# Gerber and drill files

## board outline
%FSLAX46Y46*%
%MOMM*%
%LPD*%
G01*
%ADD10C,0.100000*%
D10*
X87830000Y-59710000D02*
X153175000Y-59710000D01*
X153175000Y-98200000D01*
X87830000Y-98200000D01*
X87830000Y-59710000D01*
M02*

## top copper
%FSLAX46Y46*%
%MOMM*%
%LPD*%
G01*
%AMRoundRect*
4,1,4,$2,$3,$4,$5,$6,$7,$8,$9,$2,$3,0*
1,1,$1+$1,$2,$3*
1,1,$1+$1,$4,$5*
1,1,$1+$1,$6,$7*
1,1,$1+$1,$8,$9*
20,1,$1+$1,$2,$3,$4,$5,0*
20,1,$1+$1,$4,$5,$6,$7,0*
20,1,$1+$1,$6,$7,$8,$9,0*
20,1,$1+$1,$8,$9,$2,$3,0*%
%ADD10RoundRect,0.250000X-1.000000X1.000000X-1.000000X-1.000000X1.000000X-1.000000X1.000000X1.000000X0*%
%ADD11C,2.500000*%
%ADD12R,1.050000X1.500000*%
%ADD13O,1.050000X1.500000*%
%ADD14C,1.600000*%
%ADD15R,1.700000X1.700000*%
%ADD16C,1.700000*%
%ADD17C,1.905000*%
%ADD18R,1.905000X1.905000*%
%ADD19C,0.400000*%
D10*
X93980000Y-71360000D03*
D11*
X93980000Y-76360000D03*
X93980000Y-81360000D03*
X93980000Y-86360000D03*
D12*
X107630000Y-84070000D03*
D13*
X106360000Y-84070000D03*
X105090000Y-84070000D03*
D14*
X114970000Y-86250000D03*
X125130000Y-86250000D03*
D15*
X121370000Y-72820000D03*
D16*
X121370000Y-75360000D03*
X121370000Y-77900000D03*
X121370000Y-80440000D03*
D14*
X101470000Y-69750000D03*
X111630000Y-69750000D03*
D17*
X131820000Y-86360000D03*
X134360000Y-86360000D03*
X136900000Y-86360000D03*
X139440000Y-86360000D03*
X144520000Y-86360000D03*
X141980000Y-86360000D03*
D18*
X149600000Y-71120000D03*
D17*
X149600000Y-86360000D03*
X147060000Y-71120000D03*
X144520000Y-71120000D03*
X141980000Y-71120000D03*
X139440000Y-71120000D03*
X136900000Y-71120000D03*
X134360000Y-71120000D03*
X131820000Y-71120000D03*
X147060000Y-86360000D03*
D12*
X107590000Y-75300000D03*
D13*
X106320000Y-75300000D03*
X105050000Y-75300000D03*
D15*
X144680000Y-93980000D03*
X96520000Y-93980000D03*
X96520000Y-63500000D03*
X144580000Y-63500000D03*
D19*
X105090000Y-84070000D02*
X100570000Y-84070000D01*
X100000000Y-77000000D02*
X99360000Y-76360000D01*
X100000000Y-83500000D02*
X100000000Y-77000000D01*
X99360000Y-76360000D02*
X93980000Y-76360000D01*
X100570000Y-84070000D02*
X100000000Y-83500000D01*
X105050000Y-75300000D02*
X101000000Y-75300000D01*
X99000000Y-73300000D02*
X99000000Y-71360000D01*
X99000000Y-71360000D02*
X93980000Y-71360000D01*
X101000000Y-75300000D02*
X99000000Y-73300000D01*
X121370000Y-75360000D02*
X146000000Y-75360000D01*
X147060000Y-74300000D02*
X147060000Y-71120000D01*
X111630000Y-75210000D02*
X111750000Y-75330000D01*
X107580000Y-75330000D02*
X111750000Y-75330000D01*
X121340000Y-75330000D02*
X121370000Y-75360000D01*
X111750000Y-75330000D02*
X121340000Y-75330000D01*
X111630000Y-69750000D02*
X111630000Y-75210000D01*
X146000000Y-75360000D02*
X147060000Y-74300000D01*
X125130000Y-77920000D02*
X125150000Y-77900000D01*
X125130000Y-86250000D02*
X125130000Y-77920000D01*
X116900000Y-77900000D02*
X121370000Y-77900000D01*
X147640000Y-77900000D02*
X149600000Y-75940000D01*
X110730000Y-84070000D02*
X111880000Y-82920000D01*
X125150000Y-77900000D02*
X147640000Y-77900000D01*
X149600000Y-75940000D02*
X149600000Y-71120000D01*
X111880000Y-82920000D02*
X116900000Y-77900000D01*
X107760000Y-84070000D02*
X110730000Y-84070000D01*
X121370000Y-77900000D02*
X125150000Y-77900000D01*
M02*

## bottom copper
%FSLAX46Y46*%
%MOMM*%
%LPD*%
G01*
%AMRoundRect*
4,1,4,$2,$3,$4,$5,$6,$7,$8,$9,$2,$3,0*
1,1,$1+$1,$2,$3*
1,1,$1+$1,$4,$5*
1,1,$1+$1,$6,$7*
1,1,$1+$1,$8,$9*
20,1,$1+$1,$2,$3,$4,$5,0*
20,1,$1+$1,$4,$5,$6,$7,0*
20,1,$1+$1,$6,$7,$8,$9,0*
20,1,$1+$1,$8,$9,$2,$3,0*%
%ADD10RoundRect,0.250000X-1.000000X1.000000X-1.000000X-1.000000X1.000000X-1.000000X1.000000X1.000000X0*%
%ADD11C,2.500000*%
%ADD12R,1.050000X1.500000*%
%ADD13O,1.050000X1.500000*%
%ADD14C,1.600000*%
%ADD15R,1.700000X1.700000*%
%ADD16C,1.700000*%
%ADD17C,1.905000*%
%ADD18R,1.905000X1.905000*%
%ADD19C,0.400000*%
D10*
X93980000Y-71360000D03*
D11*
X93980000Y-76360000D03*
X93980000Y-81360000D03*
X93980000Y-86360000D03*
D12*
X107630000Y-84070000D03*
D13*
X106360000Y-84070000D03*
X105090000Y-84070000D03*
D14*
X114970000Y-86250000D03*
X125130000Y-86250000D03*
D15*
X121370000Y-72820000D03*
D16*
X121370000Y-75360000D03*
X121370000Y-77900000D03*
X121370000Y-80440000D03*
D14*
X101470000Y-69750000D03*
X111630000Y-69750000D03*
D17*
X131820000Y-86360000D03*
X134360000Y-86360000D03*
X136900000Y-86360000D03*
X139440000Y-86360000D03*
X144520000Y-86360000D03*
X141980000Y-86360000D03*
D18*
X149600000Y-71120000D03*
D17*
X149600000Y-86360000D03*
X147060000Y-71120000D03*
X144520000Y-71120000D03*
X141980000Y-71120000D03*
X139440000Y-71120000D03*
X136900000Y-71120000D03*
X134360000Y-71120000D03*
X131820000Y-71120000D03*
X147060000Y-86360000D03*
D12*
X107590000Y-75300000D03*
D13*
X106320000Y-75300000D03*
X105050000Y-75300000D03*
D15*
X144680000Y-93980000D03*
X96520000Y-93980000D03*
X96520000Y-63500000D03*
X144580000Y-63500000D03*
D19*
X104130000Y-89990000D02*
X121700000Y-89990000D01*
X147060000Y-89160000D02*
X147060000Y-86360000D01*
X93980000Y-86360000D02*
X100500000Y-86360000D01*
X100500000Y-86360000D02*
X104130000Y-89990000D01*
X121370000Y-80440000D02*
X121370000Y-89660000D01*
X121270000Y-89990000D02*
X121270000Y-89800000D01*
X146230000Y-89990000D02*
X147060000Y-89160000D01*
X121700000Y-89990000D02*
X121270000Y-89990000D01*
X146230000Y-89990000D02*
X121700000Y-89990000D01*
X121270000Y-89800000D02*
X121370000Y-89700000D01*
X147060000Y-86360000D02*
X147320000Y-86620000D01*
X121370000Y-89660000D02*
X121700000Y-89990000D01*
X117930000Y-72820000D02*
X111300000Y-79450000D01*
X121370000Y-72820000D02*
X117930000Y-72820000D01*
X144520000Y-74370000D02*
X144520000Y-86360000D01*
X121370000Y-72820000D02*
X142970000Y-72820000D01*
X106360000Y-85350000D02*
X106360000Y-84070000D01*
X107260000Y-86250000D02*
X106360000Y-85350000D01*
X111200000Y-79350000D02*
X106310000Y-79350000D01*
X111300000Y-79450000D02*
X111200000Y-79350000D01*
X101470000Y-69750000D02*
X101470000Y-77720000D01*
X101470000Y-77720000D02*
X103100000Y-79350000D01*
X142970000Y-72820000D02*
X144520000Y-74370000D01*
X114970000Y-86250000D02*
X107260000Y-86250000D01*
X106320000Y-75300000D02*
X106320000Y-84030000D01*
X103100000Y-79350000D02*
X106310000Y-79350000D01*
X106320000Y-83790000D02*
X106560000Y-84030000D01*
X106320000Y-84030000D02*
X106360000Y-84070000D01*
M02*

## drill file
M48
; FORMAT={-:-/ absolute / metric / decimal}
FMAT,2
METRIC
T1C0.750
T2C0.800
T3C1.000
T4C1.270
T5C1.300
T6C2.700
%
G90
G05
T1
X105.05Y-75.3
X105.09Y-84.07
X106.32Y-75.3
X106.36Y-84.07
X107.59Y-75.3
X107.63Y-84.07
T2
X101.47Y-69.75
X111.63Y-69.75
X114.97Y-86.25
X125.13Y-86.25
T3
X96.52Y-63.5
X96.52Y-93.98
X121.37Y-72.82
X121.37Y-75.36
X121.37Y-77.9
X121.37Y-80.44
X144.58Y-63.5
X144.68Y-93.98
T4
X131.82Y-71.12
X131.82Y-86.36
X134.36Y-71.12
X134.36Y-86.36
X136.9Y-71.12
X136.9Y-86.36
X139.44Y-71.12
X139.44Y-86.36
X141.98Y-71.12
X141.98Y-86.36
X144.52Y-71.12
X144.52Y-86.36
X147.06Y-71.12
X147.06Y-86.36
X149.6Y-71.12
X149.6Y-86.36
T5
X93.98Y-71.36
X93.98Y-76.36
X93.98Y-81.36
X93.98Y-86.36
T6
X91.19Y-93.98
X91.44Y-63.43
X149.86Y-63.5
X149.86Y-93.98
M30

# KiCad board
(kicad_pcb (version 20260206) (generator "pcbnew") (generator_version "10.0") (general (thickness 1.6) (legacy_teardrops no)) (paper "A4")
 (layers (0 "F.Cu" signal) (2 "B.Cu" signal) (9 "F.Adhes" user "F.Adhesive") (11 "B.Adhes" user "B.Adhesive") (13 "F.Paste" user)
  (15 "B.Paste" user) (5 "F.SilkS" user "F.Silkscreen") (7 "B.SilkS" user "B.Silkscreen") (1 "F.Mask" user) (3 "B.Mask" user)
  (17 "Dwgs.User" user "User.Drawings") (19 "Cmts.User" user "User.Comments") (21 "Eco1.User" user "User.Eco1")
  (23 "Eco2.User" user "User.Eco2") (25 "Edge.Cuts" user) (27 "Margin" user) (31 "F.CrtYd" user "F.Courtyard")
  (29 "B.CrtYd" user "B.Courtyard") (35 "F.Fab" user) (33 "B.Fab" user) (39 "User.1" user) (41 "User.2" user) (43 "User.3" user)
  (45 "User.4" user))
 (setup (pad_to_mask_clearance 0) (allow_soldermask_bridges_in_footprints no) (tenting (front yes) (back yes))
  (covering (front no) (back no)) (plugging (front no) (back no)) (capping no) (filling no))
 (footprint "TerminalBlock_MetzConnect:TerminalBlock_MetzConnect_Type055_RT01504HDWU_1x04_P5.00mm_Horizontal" (layer "F.Cu")
  (at 93.98 71.36 -90)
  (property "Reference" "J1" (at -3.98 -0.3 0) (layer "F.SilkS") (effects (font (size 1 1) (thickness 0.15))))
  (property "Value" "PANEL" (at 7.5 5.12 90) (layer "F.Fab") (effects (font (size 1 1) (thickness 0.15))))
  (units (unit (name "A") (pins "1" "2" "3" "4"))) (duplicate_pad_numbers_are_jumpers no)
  (pad "1" thru_hole roundrect (at 0 0 270) (size 2.5 2.5) (drill 1.3) (layers "*.Cu" "*.Mask") (remove_unused_layers no)
   (roundrect_rratio 0.1) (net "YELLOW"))
  (pad "2" thru_hole circle (at 5 0 270) (size 2.5 2.5) (drill 1.3) (layers "*.Cu" "*.Mask") (remove_unused_layers no) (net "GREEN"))
  (pad "3" thru_hole circle (at 10 0 270) (size 2.5 2.5) (drill 1.3) (layers "*.Cu" "*.Mask") (remove_unused_layers no) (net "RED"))
  (pad "4" thru_hole circle (at 15 0 270) (size 2.5 2.5) (drill 1.3) (layers "*.Cu" "*.Mask") (remove_unused_layers no) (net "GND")))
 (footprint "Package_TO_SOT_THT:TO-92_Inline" (layer "F.Cu") (at 107.63 84.07 180)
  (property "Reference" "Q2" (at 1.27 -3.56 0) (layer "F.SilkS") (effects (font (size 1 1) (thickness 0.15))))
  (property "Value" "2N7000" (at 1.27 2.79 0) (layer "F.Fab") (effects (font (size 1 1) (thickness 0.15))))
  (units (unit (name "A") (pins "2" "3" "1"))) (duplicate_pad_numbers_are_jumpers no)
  (pad "1" thru_hole rect (at 0 0 180) (size 1.05 1.5) (drill 0.75) (layers "*.Cu" "*.Mask") (remove_unused_layers no) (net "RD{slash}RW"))
  (pad "2" thru_hole oval (at 1.27 0 180) (size 1.05 1.5) (drill 0.75) (layers "*.Cu" "*.Mask") (remove_unused_layers no) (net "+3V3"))
  (pad "3" thru_hole oval (at 2.54 0 180) (size 1.05 1.5) (drill 0.75) (layers "*.Cu" "*.Mask") (remove_unused_layers no) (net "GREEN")))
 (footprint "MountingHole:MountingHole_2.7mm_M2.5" (layer "F.Cu") (at 149.86 63.5)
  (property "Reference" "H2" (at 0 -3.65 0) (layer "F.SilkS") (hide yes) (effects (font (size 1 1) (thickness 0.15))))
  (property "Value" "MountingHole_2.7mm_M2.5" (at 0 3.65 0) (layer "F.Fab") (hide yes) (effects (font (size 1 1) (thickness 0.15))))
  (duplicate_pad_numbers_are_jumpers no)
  (pad "" np_thru_hole circle (at 0 0) (size 2.7 2.7) (drill 2.7) (layers "*.Cu" "*.Mask")))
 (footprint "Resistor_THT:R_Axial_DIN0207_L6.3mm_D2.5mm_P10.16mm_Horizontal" (layer "F.Cu") (at 114.97 86.25)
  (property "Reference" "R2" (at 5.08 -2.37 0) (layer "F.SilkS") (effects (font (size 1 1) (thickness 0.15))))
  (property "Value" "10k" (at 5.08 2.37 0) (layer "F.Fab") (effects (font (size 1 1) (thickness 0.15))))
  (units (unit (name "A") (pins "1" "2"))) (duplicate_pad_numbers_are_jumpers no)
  (pad "1" thru_hole circle (at 0 0) (size 1.6 1.6) (drill 0.8) (layers "*.Cu" "*.Mask") (remove_unused_layers no) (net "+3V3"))
  (pad "2" thru_hole circle (at 10.16 0) (size 1.6 1.6) (drill 0.8) (layers "*.Cu" "*.Mask") (remove_unused_layers no) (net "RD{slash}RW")))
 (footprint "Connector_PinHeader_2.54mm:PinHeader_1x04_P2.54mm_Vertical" (layer "F.Cu") (at 121.37 72.82)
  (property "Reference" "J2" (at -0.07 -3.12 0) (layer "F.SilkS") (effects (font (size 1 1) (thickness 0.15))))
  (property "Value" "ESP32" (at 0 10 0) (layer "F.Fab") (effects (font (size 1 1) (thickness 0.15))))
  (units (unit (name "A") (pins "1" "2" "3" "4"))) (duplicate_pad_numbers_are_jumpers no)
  (pad "1" thru_hole rect (at 0 0) (size 1.7 1.7) (drill 1) (layers "*.Cu" "*.Mask") (remove_unused_layers no) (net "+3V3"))
  (pad "2" thru_hole circle (at 0 2.54) (size 1.7 1.7) (drill 1) (layers "*.Cu" "*.Mask") (remove_unused_layers no) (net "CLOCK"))
  (pad "3" thru_hole circle (at 0 5.08) (size 1.7 1.7) (drill 1) (layers "*.Cu" "*.Mask") (remove_unused_layers no) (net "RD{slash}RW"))
  (pad "4" thru_hole circle (at 0 7.62) (size 1.7 1.7) (drill 1) (layers "*.Cu" "*.Mask") (remove_unused_layers no) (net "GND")))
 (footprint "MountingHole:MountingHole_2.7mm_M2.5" (layer "F.Cu") (at 91.19 93.98)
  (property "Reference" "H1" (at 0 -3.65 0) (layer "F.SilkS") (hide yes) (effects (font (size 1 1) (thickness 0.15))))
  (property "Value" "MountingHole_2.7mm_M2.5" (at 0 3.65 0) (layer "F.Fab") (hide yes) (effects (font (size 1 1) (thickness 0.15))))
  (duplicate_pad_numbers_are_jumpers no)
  (pad "" np_thru_hole circle (at 0 0) (size 2.7 2.7) (drill 2.7) (layers "*.Cu" "*.Mask")))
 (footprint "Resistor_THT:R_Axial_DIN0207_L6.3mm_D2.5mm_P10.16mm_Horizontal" (layer "F.Cu") (at 101.47 69.75)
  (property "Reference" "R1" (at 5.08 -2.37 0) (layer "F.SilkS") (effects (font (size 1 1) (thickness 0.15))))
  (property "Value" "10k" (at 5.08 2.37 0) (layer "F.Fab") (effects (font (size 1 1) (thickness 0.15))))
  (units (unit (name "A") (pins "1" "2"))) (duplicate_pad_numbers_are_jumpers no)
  (pad "1" thru_hole circle (at 0 0) (size 1.6 1.6) (drill 0.8) (layers "*.Cu" "*.Mask") (remove_unused_layers no) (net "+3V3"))
  (pad "2" thru_hole circle (at 10.16 0) (size 1.6 1.6) (drill 0.8) (layers "*.Cu" "*.Mask") (remove_unused_layers no) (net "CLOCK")))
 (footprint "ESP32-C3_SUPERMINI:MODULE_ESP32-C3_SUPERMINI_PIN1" (layer "F.Cu") (at 139.7 78.74 -90)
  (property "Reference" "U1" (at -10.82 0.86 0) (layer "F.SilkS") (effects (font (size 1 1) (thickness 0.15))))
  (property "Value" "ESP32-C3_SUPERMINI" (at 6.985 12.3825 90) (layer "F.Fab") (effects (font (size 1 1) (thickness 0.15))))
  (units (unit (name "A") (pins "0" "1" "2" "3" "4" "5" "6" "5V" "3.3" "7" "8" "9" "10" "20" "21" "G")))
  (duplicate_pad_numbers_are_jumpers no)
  (pad "0" thru_hole circle (at 7.62 7.88 270) (size 1.905 1.905) (drill 1.27) (layers "*.Cu" "*.Mask") (remove_unused_layers no)
   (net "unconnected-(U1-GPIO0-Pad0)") (solder_mask_margin 0.102))
  (pad "1" thru_hole circle (at 7.62 5.34 270) (size 1.905 1.905) (drill 1.27) (layers "*.Cu" "*.Mask") (remove_unused_layers no)
   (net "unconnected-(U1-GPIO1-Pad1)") (solder_mask_margin 0.102))
  (pad "2" thru_hole circle (at 7.62 2.8 270) (size 1.905 1.905) (drill 1.27) (layers "*.Cu" "*.Mask") (remove_unused_layers no)
   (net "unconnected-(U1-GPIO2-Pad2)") (solder_mask_margin 0.102))
  (pad "3" thru_hole circle (at 7.62 0.26 270) (size 1.905 1.905) (drill 1.27) (layers "*.Cu" "*.Mask") (remove_unused_layers no)
   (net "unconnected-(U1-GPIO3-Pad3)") (solder_mask_margin 0.102))
  (pad "3.3" thru_hole circle (at 7.62 -4.82 270) (size 1.905 1.905) (drill 1.27) (layers "*.Cu" "*.Mask") (remove_unused_layers no)
   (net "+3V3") (solder_mask_margin 0.102))
  (pad "4" thru_hole circle (at 7.62 -2.28 270) (size 1.905 1.905) (drill 1.27) (layers "*.Cu" "*.Mask") (remove_unused_layers no)
   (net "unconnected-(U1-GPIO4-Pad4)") (solder_mask_margin 0.102))
  (pad "5" thru_hole rect (at -7.62 -9.9 270) (size 1.905 1.905) (drill 1.27) (layers "*.Cu" "*.Mask") (remove_unused_layers no)
   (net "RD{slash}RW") (solder_mask_margin 0.102))
  (pad "5V" thru_hole circle (at 7.62 -9.9 270) (size 1.905 1.905) (drill 1.27) (layers "*.Cu" "*.Mask") (remove_unused_layers no)
   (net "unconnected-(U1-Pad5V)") (solder_mask_margin 0.102))
  (pad "6" thru_hole circle (at -7.62 -7.36 270) (size 1.905 1.905) (drill 1.27) (layers "*.Cu" "*.Mask") (remove_unused_layers no)
   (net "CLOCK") (solder_mask_margin 0.102))
  (pad "7" thru_hole circle (at -7.62 -4.82 270) (size 1.905 1.905) (drill 1.27) (layers "*.Cu" "*.Mask") (remove_unused_layers no)
   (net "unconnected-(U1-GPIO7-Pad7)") (solder_mask_margin 0.102))
  (pad "8" thru_hole circle (at -7.62 -2.28 270) (size 1.905 1.905) (drill 1.27) (layers "*.Cu" "*.Mask") (remove_unused_layers no)
   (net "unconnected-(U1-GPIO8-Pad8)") (solder_mask_margin 0.102))
  (pad "9" thru_hole circle (at -7.62 0.26 270) (size 1.905 1.905) (drill 1.27) (layers "*.Cu" "*.Mask") (remove_unused_layers no)
   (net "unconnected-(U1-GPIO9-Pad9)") (solder_mask_margin 0.102))
  (pad "10" thru_hole circle (at -7.62 2.8 270) (size 1.905 1.905) (drill 1.27) (layers "*.Cu" "*.Mask") (remove_unused_layers no)
   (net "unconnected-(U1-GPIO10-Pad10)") (solder_mask_margin 0.102))
  (pad "20" thru_hole circle (at -7.62 5.34 270) (size 1.905 1.905) (drill 1.27) (layers "*.Cu" "*.Mask") (remove_unused_layers no)
   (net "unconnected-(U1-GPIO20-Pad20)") (solder_mask_margin 0.102))
  (pad "21" thru_hole circle (at -7.62 7.88 270) (size 1.905 1.905) (drill 1.27) (layers "*.Cu" "*.Mask") (remove_unused_layers no)
   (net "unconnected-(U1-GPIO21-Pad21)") (solder_mask_margin 0.102))
  (pad "G" thru_hole circle (at 7.62 -7.36 270) (size 1.905 1.905) (drill 1.27) (layers "*.Cu" "*.Mask") (remove_unused_layers no)
   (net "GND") (solder_mask_margin 0.102)))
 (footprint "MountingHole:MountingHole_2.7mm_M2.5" (layer "F.Cu") (at 91.44 63.43)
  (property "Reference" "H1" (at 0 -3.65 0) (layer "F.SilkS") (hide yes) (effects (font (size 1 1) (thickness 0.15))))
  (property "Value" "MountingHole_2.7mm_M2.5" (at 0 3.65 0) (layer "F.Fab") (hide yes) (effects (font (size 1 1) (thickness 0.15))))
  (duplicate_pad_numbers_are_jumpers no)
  (pad "" np_thru_hole circle (at 0 0) (size 2.7 2.7) (drill 2.7) (layers "*.Cu" "*.Mask")))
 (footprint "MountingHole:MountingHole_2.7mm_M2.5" (layer "F.Cu") (at 149.86 93.98)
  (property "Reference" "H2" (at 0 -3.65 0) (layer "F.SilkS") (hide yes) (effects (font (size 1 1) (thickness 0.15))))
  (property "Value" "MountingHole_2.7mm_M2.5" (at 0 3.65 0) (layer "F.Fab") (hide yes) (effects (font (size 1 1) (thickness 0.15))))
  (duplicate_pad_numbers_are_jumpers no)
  (pad "" np_thru_hole circle (at 0 0) (size 2.7 2.7) (drill 2.7) (layers "*.Cu" "*.Mask")))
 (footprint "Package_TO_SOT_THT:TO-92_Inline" (layer "F.Cu") (at 107.59 75.3 180)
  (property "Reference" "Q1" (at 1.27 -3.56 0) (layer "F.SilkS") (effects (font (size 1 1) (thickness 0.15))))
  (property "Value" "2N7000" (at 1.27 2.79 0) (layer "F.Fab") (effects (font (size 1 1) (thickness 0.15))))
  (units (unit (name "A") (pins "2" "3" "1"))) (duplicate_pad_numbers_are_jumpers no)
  (pad "1" thru_hole rect (at 0 0 180) (size 1.05 1.5) (drill 0.75) (layers "*.Cu" "*.Mask") (remove_unused_layers no) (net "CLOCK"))
  (pad "2" thru_hole oval (at 1.27 0 180) (size 1.05 1.5) (drill 0.75) (layers "*.Cu" "*.Mask") (remove_unused_layers no) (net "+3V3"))
  (pad "3" thru_hole oval (at 2.54 0 180) (size 1.05 1.5) (drill 0.75) (layers "*.Cu" "*.Mask") (remove_unused_layers no) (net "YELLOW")))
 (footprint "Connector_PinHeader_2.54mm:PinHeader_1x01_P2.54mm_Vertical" (layer "B.Cu") (at 144.68 93.98)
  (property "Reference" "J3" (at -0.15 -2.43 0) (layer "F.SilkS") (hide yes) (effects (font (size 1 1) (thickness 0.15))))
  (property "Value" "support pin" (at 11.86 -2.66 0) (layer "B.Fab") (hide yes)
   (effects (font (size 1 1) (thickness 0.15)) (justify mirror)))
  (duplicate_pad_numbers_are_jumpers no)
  (pad "1" thru_hole rect (at 0 0) (size 1.7 1.7) (drill 1) (layers "*.Cu" "*.Mask") (remove_unused_layers no)))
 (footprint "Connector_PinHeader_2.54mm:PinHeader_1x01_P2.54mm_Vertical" (layer "B.Cu") (at 96.52 93.98)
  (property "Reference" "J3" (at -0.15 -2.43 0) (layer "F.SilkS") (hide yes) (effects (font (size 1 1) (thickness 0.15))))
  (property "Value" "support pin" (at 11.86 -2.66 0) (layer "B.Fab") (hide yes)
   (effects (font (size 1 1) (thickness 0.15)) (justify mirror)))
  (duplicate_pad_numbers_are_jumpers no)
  (pad "1" thru_hole rect (at 0 0) (size 1.7 1.7) (drill 1) (layers "*.Cu" "*.Mask") (remove_unused_layers no)))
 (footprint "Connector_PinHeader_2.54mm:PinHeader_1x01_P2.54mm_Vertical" (layer "B.Cu") (at 96.52 63.5)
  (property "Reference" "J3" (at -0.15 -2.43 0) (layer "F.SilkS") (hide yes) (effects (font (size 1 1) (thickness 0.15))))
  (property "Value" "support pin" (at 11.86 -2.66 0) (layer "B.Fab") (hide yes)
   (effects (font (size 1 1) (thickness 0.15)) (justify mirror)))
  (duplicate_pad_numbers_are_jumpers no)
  (pad "1" thru_hole rect (at 0 0) (size 1.7 1.7) (drill 1) (layers "*.Cu" "*.Mask") (remove_unused_layers no)))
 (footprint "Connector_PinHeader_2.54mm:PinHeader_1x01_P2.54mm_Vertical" (layer "B.Cu") (at 144.58 63.5)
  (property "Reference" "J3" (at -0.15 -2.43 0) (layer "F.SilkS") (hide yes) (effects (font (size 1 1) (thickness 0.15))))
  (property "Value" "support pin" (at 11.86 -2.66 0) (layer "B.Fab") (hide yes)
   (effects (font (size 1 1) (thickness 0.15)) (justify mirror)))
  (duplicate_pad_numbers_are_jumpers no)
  (pad "1" thru_hole rect (at 0 0) (size 1.7 1.7) (drill 1) (layers "*.Cu" "*.Mask") (remove_unused_layers no)))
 (gr_rect (start 87.83 59.71) (end 153.175 98.2) (stroke (width 0.1) (type default)) (fill no) (layer "Edge.Cuts"))
 (segment (start 105.09 84.07) (end 100.57 84.07) (width 0.4) (layer "F.Cu") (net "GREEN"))
 (segment (start 100 77) (end 99.36 76.36) (width 0.4) (layer "F.Cu") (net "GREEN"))
 (segment (start 100 83.5) (end 100 77) (width 0.4) (layer "F.Cu") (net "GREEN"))
 (segment (start 99.36 76.36) (end 93.98 76.36) (width 0.4) (layer "F.Cu") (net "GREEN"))
 (segment (start 100.57 84.07) (end 100 83.5) (width 0.4) (layer "F.Cu") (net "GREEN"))
 (segment (start 104.13 89.99) (end 121.7 89.99) (width 0.4) (layer "B.Cu") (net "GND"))
 (segment (start 147.06 89.16) (end 147.06 86.36) (width 0.4) (layer "B.Cu") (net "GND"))
 (segment (start 93.98 86.36) (end 100.5 86.36) (width 0.4) (layer "B.Cu") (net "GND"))
 (segment (start 100.5 86.36) (end 104.13 89.99) (width 0.4) (layer "B.Cu") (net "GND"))
 (segment (start 121.37 80.44) (end 121.37 89.66) (width 0.4) (layer "B.Cu") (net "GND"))
 (segment (start 121.27 89.99) (end 121.27 89.8) (width 0.4) (layer "B.Cu") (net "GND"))
 (segment (start 146.23 89.99) (end 147.06 89.16) (width 0.4) (layer "B.Cu") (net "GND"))
 (segment (start 121.7 89.99) (end 121.27 89.99) (width 0.4) (layer "B.Cu") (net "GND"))
 (segment (start 146.23 89.99) (end 121.7 89.99) (width 0.4) (layer "B.Cu") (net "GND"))
 (segment (start 121.27 89.8) (end 121.37 89.7) (width 0.4) (layer "B.Cu") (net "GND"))
 (segment (start 147.06 86.36) (end 147.32 86.62) (width 0.4) (layer "B.Cu") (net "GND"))
 (segment (start 121.37 89.66) (end 121.7 89.99) (width 0.4) (layer "B.Cu") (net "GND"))
 (segment (start 105.05 75.3) (end 101 75.3) (width 0.4) (layer "F.Cu") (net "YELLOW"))
 (segment (start 99 73.3) (end 99 71.36) (width 0.4) (layer "F.Cu") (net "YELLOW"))
 (segment (start 99 71.36) (end 93.98 71.36) (width 0.4) (layer "F.Cu") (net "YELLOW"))
 (segment (start 101 75.3) (end 99 73.3) (width 0.4) (layer "F.Cu") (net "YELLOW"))
 (segment (start 117.93 72.82) (end 111.3 79.45) (width 0.4) (layer "B.Cu") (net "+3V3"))
 (segment (start 121.37 72.82) (end 117.93 72.82) (width 0.4) (layer "B.Cu") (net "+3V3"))
 (segment (start 144.52 74.37) (end 144.52 86.36) (width 0.4) (layer "B.Cu") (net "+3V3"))
 (segment (start 121.37 72.82) (end 142.97 72.82) (width 0.4) (layer "B.Cu") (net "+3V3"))
 (segment (start 106.36 85.35) (end 106.36 84.07) (width 0.4) (layer "B.Cu") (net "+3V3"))
 (segment (start 107.26 86.25) (end 106.36 85.35) (width 0.4) (layer "B.Cu") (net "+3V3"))
 (segment (start 111.2 79.35) (end 106.31 79.35) (width 0.4) (layer "B.Cu") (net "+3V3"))
 (segment (start 111.3 79.45) (end 111.2 79.35) (width 0.4) (layer "B.Cu") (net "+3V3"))
 (segment (start 101.47 69.75) (end 101.47 77.72) (width 0.4) (layer "B.Cu") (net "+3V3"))
 (segment (start 101.47 77.72) (end 103.1 79.35) (width 0.4) (layer "B.Cu") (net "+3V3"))
 (segment (start 142.97 72.82) (end 144.52 74.37) (width 0.4) (layer "B.Cu") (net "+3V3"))
 (segment (start 114.97 86.25) (end 107.26 86.25) (width 0.4) (layer "B.Cu") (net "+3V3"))
 (segment (start 106.32 75.3) (end 106.32 84.03) (width 0.4) (layer "B.Cu") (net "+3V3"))
 (segment (start 103.1 79.35) (end 106.31 79.35) (width 0.4) (layer "B.Cu") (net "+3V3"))
 (segment (start 106.32 83.79) (end 106.56 84.03) (width 0.4) (layer "B.Cu") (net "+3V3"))
 (segment (start 106.32 84.03) (end 106.36 84.07) (width 0.4) (layer "B.Cu") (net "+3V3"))
 (segment (start 121.37 75.36) (end 146 75.36) (width 0.4) (layer "F.Cu") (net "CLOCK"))
 (segment (start 147.06 74.3) (end 147.06 71.12) (width 0.4) (layer "F.Cu") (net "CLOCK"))
 (segment (start 111.63 75.21) (end 111.75 75.33) (width 0.4) (layer "F.Cu") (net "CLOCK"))
 (segment (start 107.58 75.33) (end 111.75 75.33) (width 0.4) (layer "F.Cu") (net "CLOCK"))
 (segment (start 121.34 75.33) (end 121.37 75.36) (width 0.4) (layer "F.Cu") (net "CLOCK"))
 (segment (start 111.75 75.33) (end 121.34 75.33) (width 0.4) (layer "F.Cu") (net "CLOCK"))
 (segment (start 111.63 69.75) (end 111.63 75.21) (width 0.4) (layer "F.Cu") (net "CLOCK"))
 (segment (start 146 75.36) (end 147.06 74.3) (width 0.4) (layer "F.Cu") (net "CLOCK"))
 (segment (start 125.13 77.92) (end 125.15 77.9) (width 0.4) (layer "F.Cu") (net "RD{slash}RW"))
 (segment (start 125.13 86.25) (end 125.13 77.92) (width 0.4) (layer "F.Cu") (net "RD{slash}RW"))
 (segment (start 116.9 77.9) (end 121.37 77.9) (width 0.4) (layer "F.Cu") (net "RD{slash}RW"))
 (segment (start 147.64 77.9) (end 149.6 75.94) (width 0.4) (layer "F.Cu") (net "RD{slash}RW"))
 (segment (start 110.73 84.07) (end 111.88 82.92) (width 0.4) (layer "F.Cu") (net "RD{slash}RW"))
 (segment (start 125.15 77.9) (end 147.64 77.9) (width 0.4) (layer "F.Cu") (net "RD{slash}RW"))
 (segment (start 149.6 75.94) (end 149.6 71.12) (width 0.4) (layer "F.Cu") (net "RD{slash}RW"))
 (segment (start 111.88 82.92) (end 116.9 77.9) (width 0.4) (layer "F.Cu") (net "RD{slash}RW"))
 (segment (start 107.76 84.07) (end 110.73 84.07) (width 0.4) (layer "F.Cu") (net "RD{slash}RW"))
 (segment (start 121.37 77.9) (end 125.15 77.9) (width 0.4) (layer "F.Cu") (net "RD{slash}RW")))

